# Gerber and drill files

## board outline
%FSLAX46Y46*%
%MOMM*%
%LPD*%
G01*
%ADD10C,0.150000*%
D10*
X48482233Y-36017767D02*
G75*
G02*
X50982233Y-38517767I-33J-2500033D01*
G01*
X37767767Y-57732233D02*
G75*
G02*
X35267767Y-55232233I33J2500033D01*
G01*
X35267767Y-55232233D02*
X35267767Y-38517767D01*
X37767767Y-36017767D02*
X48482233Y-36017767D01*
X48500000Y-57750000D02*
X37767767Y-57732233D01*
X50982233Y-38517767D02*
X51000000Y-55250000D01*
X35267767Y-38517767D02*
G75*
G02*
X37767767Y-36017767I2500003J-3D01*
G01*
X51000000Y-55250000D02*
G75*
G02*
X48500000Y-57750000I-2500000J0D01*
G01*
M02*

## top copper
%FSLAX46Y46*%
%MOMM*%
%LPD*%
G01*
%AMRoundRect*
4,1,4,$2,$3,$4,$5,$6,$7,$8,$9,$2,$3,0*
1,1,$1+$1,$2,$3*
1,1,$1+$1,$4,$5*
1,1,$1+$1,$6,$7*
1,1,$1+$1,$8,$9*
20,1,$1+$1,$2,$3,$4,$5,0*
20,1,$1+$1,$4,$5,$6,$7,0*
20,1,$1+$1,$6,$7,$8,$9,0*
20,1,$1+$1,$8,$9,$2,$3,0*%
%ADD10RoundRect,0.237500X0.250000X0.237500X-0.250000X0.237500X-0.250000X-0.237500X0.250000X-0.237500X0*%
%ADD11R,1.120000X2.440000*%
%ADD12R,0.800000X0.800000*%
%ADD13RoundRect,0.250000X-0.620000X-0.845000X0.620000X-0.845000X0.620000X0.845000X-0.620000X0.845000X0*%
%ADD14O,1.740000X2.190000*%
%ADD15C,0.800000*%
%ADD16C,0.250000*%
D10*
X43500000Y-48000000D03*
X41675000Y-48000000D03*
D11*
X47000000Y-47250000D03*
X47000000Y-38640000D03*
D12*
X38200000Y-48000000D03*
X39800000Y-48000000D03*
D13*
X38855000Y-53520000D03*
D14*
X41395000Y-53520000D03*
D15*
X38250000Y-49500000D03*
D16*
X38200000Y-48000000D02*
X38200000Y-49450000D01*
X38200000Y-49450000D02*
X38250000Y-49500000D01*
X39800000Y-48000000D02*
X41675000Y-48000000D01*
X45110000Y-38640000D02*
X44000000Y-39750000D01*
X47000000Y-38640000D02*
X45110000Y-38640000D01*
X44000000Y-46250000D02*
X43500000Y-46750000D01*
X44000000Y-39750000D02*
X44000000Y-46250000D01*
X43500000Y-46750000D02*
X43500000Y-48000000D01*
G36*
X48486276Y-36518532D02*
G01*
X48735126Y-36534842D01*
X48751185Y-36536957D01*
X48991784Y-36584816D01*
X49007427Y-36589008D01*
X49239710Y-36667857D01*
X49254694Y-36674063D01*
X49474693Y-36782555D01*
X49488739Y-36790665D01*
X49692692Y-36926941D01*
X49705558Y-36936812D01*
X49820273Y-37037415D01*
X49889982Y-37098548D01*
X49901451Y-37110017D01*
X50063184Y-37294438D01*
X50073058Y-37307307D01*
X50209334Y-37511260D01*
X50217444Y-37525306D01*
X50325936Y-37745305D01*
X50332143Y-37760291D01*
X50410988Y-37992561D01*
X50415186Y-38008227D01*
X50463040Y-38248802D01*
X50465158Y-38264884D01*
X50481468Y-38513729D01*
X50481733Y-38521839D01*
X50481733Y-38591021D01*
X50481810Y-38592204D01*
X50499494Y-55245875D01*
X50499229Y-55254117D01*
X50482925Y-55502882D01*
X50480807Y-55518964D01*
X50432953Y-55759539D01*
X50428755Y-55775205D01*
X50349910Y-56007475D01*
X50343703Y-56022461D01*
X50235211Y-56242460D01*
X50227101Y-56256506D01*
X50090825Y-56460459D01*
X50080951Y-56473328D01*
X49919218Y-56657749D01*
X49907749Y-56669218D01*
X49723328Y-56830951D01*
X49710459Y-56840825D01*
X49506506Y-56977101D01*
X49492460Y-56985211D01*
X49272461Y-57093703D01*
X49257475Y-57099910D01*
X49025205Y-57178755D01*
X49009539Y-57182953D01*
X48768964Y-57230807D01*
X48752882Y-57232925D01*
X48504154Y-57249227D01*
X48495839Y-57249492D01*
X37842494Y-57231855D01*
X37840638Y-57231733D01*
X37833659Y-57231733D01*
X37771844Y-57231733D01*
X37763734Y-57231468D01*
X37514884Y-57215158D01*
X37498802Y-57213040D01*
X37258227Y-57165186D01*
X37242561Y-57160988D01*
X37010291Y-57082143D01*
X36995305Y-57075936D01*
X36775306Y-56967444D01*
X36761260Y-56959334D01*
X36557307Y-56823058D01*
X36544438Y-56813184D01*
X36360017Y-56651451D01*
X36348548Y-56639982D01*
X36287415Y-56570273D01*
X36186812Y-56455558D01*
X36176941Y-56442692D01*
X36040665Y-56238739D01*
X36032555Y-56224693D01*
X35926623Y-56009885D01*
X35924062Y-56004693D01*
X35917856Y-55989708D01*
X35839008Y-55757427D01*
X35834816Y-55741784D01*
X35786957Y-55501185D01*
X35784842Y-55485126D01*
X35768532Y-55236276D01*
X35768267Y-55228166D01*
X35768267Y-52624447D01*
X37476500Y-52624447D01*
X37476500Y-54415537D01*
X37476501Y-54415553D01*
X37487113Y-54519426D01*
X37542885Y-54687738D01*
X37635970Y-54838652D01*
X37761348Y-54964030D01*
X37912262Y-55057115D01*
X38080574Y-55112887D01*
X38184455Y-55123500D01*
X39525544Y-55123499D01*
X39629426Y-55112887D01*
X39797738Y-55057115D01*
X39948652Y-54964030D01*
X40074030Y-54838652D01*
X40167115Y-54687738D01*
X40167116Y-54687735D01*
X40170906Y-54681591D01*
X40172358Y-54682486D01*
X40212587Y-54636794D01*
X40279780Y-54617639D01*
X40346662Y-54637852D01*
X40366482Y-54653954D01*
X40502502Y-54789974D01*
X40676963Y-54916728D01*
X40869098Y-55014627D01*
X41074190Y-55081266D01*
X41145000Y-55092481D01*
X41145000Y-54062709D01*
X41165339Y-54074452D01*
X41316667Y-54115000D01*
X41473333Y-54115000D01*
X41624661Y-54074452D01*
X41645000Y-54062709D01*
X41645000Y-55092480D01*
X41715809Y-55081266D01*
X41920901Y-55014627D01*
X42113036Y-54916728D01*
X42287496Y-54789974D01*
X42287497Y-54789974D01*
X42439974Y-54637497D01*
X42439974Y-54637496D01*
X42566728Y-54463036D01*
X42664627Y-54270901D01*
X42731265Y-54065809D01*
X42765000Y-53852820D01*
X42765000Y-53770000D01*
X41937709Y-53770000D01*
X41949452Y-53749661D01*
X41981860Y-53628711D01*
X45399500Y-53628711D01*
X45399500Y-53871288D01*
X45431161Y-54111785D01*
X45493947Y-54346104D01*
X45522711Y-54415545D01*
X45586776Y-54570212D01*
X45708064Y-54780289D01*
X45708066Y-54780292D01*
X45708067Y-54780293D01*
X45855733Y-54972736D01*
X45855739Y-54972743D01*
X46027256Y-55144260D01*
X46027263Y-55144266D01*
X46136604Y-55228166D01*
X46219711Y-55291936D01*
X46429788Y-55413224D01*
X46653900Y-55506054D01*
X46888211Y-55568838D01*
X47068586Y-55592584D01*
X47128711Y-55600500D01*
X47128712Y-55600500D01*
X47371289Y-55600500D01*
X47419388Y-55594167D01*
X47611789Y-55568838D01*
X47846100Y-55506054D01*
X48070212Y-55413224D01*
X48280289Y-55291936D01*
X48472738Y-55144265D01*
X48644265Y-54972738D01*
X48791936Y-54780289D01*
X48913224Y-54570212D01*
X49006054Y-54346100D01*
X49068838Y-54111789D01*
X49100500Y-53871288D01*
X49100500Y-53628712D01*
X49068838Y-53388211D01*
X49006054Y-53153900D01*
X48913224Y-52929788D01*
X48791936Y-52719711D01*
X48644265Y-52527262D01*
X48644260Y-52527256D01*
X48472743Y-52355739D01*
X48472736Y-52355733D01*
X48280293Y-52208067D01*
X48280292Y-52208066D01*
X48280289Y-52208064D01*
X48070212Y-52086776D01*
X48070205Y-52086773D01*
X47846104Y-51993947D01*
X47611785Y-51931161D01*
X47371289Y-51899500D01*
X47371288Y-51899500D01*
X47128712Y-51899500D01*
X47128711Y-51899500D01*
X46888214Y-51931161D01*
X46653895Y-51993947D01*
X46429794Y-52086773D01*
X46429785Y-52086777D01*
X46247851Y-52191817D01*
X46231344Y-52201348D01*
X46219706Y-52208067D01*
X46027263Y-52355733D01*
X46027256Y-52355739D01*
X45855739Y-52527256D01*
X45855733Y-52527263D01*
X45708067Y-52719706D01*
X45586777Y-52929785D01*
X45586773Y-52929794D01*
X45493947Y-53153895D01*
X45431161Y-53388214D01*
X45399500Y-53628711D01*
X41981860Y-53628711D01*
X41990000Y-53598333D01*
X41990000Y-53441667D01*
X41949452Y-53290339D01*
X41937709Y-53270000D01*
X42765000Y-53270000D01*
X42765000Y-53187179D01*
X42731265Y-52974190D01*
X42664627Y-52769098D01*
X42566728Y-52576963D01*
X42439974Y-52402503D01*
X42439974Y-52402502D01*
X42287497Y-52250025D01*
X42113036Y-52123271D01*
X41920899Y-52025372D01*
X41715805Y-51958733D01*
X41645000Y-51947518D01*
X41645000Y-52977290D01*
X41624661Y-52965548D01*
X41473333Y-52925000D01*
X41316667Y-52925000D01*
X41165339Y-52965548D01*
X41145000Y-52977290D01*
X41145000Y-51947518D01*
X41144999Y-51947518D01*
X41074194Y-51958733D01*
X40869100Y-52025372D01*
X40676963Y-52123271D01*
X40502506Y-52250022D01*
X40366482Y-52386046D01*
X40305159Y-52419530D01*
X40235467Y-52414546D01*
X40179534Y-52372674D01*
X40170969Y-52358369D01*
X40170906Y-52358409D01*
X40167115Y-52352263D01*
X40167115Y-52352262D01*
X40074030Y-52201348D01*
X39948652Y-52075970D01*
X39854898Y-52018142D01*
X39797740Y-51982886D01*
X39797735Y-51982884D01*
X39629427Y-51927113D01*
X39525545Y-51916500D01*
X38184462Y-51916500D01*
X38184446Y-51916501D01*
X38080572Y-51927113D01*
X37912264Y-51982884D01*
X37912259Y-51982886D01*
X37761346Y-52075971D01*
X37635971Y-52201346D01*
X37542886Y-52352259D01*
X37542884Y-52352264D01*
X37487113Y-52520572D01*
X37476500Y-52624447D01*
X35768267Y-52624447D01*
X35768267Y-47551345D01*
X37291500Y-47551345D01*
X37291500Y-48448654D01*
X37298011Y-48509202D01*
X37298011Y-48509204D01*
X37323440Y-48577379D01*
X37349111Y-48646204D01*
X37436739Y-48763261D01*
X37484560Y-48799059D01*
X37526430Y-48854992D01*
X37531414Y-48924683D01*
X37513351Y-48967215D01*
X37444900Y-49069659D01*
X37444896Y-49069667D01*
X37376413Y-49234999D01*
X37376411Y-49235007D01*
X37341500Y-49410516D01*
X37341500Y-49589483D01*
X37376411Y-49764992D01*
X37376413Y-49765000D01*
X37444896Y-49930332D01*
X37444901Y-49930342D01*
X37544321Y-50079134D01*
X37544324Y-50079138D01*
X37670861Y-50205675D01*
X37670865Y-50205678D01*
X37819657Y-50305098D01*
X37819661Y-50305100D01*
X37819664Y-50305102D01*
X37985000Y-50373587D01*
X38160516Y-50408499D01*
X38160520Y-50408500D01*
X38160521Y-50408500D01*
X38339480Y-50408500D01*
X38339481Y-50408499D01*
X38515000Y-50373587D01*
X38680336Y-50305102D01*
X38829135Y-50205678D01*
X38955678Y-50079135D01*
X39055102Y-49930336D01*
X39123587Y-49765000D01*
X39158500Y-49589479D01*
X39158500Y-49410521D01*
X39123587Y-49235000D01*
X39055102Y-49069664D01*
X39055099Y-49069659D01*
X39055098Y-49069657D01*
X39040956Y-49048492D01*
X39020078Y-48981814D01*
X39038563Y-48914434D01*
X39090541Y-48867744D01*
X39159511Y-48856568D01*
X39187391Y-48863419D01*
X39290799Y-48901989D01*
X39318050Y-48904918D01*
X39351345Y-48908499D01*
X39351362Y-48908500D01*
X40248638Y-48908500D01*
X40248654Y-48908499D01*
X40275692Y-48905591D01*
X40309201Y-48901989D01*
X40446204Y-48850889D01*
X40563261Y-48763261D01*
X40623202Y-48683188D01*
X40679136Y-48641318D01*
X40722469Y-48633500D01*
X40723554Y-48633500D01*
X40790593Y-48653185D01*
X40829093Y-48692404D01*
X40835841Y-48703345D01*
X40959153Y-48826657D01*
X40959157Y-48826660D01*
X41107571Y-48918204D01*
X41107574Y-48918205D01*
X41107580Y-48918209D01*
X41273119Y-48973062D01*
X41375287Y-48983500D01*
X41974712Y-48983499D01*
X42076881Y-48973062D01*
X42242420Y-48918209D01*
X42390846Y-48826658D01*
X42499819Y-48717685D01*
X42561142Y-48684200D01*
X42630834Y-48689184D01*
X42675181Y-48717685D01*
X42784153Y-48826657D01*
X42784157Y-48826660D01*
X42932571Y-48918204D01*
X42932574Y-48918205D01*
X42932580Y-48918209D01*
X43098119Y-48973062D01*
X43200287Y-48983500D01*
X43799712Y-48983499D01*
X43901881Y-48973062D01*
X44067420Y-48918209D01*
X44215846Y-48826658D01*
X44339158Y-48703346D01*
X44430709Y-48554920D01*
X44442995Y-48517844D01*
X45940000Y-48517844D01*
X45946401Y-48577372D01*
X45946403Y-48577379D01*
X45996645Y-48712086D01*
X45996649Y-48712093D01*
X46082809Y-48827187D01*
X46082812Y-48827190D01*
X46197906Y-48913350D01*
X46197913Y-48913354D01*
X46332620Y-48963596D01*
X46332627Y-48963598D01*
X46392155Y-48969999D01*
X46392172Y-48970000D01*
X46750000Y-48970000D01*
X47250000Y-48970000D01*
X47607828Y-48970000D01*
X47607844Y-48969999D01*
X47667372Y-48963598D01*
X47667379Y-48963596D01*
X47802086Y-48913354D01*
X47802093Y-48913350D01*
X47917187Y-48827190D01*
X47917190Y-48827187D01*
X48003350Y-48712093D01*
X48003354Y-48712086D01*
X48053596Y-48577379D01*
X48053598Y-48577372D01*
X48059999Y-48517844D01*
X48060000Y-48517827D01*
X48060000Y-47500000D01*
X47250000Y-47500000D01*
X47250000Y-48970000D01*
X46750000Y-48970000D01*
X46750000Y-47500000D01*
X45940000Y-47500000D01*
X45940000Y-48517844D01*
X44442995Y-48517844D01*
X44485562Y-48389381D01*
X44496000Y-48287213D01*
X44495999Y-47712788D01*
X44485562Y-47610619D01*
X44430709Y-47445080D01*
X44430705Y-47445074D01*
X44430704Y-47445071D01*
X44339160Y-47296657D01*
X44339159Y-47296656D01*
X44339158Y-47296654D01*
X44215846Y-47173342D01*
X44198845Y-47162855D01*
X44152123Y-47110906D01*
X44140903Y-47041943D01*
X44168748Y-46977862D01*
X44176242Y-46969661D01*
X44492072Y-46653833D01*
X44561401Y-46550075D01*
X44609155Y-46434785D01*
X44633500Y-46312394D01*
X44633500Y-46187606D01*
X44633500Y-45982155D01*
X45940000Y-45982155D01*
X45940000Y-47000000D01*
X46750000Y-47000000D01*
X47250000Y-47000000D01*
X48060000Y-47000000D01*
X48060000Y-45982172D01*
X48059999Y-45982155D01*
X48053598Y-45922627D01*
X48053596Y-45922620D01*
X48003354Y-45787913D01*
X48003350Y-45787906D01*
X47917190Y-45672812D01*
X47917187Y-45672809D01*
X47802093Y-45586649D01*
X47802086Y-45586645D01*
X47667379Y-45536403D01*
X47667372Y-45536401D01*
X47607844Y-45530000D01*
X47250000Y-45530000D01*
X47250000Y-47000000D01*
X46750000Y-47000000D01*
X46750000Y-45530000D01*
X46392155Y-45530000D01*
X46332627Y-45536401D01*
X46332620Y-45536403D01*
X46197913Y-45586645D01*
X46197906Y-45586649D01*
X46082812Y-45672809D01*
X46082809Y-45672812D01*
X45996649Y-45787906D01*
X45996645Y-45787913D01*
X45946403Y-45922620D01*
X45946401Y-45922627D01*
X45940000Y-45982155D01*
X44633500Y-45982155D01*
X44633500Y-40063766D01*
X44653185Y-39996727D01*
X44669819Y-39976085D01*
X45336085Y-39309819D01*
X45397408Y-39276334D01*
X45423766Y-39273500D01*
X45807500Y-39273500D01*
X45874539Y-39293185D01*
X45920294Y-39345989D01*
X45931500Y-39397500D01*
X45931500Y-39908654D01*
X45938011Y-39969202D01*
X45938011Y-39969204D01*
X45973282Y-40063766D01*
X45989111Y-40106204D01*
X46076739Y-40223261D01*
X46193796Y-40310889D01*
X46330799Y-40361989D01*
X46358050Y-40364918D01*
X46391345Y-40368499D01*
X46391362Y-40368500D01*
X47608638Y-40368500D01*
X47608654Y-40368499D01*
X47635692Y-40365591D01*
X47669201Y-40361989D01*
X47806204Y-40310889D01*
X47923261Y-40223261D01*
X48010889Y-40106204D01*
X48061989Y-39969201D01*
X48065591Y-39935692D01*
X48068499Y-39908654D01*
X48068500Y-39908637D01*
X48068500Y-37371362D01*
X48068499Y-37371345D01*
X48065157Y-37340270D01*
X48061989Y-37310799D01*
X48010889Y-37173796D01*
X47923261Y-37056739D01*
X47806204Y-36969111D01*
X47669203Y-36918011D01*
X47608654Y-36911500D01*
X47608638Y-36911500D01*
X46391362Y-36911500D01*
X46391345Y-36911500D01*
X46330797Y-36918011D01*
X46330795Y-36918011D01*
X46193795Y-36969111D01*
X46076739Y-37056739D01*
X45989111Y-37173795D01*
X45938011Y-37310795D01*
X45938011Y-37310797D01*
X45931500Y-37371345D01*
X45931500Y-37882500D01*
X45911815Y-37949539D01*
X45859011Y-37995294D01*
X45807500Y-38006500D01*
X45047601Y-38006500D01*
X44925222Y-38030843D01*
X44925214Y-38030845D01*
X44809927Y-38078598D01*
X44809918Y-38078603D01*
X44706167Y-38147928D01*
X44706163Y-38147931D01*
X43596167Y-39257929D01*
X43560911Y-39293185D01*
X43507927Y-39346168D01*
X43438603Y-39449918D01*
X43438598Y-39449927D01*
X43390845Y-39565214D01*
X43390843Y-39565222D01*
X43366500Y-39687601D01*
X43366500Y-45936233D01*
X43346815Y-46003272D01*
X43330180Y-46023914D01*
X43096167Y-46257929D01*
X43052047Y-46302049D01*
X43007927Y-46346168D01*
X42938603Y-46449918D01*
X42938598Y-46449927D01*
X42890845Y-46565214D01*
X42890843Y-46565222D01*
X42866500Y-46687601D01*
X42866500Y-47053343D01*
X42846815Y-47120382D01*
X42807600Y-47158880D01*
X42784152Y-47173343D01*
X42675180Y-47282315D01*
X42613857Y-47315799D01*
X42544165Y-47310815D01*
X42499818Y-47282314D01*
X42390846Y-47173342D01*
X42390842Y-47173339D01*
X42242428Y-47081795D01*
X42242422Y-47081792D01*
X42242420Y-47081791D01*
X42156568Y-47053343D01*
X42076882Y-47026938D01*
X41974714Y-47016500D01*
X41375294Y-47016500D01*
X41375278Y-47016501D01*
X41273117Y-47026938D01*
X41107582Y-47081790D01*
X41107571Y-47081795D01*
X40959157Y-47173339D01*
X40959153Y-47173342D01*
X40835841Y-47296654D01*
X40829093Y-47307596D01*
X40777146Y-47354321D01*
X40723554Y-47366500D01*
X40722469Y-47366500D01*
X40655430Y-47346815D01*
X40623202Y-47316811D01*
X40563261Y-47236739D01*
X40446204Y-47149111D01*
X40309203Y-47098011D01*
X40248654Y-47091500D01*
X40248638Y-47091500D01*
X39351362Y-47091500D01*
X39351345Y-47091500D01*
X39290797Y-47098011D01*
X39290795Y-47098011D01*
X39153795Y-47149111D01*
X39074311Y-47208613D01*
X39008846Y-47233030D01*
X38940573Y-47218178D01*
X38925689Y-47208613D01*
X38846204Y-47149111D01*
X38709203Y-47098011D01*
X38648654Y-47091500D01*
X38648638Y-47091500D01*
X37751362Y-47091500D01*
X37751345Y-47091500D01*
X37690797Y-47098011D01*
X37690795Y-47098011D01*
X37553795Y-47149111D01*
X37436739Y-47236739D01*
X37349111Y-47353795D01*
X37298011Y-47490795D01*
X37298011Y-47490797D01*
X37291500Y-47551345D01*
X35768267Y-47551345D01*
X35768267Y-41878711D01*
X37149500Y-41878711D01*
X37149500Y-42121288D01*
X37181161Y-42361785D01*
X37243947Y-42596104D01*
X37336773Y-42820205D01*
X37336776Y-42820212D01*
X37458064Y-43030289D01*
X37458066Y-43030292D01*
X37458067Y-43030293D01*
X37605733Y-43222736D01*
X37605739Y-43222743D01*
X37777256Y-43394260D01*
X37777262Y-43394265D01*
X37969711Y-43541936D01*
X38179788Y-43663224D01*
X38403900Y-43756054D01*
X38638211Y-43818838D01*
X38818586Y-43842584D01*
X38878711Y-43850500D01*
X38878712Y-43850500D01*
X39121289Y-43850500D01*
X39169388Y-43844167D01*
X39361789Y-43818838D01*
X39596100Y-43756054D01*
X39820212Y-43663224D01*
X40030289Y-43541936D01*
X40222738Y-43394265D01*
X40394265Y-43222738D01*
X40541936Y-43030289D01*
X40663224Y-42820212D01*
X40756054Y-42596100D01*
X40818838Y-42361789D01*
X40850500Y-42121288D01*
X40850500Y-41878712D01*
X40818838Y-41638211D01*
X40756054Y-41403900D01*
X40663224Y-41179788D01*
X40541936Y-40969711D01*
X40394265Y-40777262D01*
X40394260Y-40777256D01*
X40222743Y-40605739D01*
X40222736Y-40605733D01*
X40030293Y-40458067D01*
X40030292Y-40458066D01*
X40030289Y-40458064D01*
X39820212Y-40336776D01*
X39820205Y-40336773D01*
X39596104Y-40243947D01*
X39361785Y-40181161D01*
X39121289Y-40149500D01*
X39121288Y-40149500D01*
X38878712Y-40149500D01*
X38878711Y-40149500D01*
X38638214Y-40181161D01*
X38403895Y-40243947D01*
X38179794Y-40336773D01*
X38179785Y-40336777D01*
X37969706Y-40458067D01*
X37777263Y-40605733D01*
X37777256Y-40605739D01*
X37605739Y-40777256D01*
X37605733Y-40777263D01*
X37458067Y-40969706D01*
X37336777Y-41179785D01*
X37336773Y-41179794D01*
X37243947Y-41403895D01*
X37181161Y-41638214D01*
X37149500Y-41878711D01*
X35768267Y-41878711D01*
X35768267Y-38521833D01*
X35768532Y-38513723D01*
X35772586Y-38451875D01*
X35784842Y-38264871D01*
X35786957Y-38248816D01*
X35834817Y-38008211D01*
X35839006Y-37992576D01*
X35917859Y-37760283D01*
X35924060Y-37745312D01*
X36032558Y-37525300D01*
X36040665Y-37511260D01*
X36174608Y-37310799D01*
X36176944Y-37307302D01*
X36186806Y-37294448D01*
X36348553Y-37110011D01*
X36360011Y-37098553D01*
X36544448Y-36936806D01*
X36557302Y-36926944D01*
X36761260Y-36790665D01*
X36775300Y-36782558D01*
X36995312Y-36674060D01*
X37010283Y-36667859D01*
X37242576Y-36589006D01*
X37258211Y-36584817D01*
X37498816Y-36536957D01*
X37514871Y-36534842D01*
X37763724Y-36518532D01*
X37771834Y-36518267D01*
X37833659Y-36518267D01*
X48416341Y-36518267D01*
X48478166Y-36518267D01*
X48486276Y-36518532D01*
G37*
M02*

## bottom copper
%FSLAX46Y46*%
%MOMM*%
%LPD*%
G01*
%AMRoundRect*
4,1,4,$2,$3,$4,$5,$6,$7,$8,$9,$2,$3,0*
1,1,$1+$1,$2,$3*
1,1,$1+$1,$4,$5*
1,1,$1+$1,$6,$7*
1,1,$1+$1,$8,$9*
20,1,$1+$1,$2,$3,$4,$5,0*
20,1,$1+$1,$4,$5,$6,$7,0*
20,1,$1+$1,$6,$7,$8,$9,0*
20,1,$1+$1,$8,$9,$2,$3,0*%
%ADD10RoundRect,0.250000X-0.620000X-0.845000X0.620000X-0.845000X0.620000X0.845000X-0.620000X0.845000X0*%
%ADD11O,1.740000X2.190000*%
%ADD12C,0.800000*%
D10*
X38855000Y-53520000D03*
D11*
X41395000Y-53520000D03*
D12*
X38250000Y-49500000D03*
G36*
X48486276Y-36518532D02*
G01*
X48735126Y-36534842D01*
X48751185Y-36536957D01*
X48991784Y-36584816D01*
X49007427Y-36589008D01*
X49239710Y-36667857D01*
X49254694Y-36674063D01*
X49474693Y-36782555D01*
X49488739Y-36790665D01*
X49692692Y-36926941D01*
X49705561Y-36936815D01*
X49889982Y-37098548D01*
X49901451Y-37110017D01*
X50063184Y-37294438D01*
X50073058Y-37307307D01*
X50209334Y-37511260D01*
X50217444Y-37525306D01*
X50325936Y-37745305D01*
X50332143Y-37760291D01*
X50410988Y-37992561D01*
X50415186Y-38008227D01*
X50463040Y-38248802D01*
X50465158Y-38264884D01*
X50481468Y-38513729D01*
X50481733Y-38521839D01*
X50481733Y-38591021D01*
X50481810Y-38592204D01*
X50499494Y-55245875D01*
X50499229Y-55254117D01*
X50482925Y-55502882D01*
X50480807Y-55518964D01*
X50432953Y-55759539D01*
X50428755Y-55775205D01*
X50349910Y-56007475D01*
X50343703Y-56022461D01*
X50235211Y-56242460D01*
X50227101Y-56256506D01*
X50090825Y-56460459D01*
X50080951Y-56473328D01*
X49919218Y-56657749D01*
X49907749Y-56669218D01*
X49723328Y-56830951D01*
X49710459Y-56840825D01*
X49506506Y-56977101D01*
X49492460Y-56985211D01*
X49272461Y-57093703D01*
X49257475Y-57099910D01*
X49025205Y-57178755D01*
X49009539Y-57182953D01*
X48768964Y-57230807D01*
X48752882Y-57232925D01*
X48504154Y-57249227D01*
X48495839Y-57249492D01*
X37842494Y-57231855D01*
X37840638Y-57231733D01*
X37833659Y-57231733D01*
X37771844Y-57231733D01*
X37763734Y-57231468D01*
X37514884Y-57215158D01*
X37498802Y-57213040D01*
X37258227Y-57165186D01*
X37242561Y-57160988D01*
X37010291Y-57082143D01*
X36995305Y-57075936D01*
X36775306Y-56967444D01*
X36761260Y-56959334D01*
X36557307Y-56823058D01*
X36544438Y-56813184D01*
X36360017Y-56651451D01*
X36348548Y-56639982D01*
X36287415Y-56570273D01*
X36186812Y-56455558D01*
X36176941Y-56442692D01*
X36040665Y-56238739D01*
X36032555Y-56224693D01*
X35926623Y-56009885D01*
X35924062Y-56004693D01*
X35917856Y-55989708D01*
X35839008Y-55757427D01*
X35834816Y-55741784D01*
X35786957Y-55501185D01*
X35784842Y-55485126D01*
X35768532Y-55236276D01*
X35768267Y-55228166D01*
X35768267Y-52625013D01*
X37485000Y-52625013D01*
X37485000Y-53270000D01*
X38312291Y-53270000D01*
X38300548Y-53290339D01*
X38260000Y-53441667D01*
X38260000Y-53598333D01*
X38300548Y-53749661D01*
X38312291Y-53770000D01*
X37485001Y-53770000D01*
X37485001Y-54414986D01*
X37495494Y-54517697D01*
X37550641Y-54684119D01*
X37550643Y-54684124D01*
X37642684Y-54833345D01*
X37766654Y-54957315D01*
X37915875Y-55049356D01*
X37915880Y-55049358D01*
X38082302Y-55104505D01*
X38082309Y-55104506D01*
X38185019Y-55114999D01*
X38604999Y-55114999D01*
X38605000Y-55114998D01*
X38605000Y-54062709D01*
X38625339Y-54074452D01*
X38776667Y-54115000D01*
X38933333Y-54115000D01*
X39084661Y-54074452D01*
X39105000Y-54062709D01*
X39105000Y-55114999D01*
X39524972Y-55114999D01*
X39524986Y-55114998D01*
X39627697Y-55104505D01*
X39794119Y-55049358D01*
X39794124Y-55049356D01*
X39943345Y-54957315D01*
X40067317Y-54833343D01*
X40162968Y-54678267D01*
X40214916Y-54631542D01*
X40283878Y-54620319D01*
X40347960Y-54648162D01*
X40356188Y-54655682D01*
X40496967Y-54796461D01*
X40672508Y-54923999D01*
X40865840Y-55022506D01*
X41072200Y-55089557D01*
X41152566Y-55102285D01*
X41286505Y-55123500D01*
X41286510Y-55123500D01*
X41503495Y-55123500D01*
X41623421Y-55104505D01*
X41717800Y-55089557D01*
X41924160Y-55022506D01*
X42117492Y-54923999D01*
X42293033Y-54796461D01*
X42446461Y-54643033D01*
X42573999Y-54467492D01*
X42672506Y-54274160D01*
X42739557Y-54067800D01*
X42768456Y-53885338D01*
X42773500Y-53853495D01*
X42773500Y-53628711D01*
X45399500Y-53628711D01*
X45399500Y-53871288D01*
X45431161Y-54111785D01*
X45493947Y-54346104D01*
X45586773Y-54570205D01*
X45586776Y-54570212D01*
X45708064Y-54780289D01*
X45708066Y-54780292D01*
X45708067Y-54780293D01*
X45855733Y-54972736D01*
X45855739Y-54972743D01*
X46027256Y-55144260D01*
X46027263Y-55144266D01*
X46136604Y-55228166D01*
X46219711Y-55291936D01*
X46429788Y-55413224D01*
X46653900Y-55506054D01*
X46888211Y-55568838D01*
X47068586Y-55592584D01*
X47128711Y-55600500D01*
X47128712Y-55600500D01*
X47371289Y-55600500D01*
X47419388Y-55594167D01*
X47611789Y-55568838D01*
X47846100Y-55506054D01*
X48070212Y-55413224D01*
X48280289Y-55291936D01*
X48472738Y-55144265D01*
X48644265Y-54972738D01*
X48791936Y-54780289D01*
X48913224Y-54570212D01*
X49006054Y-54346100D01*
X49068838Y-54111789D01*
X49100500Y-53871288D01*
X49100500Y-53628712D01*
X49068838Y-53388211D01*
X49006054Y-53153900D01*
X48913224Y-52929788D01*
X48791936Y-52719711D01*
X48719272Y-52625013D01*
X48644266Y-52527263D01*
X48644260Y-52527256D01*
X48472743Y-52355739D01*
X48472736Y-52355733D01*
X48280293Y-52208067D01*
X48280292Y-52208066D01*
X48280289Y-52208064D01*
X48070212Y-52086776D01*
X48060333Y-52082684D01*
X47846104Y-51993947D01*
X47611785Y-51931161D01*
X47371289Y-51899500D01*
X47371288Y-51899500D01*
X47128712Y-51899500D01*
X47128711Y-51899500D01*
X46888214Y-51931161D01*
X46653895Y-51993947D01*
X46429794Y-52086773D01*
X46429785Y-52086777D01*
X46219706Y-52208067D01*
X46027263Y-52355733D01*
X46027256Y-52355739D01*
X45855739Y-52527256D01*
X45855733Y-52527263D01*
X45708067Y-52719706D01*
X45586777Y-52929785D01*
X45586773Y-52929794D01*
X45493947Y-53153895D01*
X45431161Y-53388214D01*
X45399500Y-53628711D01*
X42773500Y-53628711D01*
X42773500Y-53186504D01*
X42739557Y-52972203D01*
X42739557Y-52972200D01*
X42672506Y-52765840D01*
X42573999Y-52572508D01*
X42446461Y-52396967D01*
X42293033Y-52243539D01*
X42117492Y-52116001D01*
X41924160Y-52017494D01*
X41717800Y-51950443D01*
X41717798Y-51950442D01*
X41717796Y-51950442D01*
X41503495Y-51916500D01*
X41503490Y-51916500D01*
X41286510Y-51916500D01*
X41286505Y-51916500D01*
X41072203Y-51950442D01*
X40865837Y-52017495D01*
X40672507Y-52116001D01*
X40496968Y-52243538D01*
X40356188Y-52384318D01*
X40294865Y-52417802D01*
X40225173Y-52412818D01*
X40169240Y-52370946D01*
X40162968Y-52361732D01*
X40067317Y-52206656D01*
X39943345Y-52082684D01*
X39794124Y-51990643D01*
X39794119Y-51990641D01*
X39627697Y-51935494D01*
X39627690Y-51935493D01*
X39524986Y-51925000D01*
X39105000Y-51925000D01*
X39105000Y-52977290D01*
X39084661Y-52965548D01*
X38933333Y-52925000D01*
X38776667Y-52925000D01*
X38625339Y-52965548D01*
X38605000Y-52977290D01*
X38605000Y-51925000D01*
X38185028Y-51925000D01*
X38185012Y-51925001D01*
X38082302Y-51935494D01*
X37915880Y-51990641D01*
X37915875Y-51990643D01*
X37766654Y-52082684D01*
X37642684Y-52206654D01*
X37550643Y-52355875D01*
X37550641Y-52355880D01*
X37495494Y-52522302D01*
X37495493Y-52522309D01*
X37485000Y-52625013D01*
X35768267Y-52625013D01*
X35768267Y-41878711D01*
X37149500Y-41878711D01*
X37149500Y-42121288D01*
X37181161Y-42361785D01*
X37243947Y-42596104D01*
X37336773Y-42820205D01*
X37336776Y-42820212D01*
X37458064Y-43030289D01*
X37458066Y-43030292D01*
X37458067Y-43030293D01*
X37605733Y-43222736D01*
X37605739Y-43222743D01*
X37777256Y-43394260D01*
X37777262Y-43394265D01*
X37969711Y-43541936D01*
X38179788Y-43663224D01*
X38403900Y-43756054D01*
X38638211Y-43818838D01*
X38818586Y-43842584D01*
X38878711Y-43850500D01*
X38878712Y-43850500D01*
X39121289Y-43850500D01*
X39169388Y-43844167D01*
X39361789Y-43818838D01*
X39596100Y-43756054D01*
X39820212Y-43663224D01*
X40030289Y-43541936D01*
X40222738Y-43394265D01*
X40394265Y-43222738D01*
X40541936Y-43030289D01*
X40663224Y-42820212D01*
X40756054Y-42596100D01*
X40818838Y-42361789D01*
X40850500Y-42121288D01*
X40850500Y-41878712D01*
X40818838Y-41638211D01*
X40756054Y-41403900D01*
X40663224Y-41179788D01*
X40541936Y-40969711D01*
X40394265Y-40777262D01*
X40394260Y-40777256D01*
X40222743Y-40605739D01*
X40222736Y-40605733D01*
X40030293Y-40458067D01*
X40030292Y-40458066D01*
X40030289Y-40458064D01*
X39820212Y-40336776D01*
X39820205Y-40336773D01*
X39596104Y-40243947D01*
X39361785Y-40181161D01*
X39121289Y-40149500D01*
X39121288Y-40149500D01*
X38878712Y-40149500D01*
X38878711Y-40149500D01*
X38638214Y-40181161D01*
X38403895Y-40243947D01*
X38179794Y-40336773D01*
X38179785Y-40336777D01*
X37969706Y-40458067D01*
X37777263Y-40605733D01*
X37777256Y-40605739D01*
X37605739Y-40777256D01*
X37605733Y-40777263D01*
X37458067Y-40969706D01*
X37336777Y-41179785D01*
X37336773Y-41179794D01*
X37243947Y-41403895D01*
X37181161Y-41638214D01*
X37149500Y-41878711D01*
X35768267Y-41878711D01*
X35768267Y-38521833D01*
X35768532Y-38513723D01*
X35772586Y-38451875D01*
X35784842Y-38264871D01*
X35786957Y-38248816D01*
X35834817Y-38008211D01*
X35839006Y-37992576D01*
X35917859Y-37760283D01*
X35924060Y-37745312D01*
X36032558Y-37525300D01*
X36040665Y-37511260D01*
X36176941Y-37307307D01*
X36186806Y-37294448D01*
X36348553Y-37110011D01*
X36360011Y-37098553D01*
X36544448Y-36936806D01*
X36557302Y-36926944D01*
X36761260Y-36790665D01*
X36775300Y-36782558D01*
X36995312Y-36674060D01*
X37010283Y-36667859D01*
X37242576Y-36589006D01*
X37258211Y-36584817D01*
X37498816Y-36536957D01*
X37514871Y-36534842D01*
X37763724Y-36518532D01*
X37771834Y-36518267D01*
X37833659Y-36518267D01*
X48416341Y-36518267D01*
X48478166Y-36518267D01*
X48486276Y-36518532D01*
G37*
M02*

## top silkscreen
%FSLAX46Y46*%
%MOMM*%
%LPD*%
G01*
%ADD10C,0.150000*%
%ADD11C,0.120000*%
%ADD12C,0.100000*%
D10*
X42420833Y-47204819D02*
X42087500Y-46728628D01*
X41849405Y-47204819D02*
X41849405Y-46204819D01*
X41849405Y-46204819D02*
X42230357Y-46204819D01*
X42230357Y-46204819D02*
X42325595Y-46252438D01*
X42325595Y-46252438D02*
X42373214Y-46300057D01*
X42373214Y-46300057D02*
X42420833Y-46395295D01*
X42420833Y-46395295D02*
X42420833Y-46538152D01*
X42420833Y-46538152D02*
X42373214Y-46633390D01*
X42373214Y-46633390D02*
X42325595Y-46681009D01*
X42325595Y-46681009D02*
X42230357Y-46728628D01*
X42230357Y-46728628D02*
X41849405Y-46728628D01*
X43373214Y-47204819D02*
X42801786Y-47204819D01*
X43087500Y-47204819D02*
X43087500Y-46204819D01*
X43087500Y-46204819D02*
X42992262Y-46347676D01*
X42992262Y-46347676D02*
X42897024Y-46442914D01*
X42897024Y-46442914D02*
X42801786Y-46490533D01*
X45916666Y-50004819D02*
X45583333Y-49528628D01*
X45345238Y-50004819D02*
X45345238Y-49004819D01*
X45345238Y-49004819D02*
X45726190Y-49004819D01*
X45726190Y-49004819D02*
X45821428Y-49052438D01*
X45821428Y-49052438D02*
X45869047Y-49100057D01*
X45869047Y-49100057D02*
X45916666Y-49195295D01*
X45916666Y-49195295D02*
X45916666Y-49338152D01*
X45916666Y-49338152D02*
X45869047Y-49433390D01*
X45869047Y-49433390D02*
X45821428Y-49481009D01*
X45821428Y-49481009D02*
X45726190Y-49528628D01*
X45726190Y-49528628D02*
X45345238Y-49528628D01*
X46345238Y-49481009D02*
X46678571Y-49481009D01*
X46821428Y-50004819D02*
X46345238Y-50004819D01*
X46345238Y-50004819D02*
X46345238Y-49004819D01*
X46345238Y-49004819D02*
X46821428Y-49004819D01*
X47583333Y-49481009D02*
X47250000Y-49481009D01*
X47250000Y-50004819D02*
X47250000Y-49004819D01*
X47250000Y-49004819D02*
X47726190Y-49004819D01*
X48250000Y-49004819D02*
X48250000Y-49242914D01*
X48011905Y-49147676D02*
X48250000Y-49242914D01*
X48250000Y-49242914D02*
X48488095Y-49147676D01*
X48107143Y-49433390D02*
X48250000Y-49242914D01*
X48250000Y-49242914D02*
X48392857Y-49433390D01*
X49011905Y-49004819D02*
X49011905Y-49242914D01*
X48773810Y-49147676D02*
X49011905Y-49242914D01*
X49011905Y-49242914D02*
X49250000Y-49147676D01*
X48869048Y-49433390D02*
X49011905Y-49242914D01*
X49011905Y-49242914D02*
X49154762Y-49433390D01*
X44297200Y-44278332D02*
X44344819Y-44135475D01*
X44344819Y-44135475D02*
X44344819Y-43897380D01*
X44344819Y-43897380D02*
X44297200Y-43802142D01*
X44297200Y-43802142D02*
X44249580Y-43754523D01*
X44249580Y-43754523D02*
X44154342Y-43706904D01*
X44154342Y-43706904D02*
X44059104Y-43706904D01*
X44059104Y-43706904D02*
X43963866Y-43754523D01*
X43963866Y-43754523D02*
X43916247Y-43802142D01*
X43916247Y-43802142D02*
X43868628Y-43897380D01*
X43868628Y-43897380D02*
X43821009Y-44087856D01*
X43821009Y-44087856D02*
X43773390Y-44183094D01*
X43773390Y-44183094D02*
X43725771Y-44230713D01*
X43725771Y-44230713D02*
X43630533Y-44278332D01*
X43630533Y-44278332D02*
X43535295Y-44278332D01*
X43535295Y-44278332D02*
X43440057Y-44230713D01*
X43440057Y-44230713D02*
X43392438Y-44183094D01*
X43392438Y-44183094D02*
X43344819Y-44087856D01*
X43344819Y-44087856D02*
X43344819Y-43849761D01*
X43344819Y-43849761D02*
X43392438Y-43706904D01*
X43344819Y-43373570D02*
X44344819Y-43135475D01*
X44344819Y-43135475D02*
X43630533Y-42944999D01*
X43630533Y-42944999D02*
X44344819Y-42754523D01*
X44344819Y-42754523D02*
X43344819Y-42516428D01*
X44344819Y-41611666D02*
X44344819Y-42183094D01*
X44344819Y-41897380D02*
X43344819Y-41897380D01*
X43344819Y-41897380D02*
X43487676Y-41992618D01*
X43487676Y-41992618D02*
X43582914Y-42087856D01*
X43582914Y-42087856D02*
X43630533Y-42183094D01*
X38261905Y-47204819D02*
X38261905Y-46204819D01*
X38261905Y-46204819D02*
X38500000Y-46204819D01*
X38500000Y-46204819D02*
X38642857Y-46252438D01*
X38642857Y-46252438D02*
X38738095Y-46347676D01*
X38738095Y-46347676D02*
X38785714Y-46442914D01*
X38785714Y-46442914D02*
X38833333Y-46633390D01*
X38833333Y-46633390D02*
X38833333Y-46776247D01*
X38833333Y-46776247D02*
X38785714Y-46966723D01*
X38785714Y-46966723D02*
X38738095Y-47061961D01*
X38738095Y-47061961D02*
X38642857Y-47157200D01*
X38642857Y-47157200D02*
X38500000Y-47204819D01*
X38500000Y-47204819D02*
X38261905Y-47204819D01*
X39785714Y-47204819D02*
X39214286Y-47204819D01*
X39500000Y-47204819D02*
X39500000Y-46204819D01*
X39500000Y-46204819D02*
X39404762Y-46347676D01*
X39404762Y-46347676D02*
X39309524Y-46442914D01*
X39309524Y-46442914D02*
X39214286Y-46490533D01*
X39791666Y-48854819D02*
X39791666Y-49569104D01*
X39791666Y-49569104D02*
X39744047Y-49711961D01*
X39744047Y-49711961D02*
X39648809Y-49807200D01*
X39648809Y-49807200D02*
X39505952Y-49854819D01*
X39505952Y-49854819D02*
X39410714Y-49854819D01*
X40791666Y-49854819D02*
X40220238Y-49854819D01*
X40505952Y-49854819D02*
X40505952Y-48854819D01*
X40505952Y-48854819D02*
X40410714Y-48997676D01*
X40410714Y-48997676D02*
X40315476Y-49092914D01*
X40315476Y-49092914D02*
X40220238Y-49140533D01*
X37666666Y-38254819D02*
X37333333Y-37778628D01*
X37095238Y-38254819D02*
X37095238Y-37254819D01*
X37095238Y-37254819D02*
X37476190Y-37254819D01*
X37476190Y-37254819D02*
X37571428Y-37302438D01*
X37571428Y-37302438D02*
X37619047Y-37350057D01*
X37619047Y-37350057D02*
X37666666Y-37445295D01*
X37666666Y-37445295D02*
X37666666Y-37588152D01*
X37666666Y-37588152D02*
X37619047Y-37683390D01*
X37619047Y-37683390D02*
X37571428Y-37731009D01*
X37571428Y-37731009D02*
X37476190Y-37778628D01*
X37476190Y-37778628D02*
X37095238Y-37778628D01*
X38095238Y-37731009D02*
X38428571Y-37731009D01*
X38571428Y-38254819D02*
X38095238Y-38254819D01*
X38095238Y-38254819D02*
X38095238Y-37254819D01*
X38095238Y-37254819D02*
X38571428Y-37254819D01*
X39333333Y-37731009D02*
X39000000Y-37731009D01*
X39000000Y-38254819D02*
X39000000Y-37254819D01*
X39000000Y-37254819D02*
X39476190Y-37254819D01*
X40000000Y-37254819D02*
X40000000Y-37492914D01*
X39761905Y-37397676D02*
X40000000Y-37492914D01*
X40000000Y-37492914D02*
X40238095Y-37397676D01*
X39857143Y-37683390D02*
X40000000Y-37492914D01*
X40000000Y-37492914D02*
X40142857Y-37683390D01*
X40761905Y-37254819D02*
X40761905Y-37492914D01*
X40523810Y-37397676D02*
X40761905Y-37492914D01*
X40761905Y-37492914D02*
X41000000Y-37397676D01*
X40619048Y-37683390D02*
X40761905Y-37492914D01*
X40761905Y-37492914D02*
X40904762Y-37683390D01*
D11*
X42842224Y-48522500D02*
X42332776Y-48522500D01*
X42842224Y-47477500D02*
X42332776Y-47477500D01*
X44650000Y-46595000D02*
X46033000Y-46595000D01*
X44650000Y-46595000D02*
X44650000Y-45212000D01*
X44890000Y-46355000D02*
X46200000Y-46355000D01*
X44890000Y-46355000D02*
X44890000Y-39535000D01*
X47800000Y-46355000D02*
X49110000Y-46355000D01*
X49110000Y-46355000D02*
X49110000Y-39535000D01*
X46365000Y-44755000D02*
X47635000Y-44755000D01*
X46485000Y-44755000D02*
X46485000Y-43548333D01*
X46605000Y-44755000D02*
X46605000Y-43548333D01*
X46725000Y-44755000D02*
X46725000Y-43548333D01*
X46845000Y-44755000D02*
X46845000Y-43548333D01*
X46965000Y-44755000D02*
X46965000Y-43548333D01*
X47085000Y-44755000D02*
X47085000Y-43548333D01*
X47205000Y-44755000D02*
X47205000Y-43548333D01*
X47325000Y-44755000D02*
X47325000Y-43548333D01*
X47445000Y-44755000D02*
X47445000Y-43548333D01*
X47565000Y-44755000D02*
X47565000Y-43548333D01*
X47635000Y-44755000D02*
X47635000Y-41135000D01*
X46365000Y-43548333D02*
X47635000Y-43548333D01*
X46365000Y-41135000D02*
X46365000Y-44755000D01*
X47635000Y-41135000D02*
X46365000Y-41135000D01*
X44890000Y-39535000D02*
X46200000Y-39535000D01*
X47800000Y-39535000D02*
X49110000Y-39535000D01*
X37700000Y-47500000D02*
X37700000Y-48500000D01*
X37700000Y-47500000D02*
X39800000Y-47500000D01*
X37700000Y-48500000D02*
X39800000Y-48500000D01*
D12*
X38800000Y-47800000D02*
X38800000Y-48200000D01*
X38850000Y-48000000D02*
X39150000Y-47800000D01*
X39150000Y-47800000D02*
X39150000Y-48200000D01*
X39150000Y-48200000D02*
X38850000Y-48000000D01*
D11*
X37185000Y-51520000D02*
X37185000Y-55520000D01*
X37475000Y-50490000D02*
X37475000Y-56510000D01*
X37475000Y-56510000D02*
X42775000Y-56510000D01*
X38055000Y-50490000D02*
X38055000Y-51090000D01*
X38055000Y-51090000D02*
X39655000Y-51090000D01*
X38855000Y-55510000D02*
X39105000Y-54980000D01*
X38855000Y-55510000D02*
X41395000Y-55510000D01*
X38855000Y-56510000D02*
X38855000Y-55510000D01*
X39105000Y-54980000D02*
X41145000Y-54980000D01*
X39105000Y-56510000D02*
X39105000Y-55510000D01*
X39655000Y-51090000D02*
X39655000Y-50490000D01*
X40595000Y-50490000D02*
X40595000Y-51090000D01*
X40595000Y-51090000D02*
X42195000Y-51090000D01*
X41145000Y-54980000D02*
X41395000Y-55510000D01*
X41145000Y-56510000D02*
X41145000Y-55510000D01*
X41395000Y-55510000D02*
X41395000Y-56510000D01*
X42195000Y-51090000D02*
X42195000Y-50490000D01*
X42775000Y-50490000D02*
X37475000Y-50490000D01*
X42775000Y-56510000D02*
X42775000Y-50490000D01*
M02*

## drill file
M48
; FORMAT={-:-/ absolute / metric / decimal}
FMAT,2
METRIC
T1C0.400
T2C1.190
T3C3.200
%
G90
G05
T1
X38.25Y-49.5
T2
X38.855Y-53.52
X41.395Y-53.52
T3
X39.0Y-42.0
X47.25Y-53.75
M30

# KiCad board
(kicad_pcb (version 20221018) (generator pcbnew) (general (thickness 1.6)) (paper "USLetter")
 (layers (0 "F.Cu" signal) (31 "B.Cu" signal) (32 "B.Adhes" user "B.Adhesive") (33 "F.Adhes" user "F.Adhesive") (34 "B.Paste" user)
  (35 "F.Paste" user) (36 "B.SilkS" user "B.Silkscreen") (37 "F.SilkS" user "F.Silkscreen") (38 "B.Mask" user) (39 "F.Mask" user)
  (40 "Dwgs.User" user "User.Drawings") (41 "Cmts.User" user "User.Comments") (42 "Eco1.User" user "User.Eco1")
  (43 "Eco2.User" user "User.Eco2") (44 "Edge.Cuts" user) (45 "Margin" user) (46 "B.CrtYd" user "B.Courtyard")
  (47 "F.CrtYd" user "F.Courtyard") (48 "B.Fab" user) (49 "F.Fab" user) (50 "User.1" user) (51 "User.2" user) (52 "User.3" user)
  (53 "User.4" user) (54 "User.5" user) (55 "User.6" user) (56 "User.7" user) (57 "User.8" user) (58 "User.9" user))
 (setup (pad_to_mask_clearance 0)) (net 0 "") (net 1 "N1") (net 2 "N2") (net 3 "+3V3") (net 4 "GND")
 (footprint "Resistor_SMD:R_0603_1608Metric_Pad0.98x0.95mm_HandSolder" (layer "F.Cu") (at 42.5875 48 180)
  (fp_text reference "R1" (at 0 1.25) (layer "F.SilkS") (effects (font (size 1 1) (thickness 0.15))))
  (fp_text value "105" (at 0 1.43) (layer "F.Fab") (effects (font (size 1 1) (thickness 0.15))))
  (fp_line (start -0.254724 -0.5225) (end 0.254724 -0.5225) (stroke (width 0.12) (type solid)) (layer "F.SilkS"))
  (fp_line (start -0.254724 0.5225) (end 0.254724 0.5225) (stroke (width 0.12) (type solid)) (layer "F.SilkS"))
  (pad "1" smd roundrect (at -0.9125 0 180) (size 0.975 0.95) (layers "F.Cu" "F.Paste" "F.Mask") (roundrect_rratio 0.25) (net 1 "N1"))
  (pad "2" smd roundrect (at 0.9125 0 180) (size 0.975 0.95) (layers "F.Cu" "F.Paste" "F.Mask") (roundrect_rratio 0.25) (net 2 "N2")))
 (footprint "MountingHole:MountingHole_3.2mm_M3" (layer "F.Cu") (at 47.25 53.75)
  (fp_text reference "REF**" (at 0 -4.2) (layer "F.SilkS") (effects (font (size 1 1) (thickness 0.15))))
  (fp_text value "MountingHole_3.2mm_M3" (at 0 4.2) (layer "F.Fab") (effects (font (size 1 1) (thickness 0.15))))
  (pad "" np_thru_hole circle (at 0 0) (size 3.2 3.2) (drill 3.2) (layers "F&B.Cu" "*.Mask")))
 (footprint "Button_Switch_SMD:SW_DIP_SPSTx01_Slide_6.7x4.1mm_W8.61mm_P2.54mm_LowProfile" (layer "F.Cu") (at 47 42.945 90)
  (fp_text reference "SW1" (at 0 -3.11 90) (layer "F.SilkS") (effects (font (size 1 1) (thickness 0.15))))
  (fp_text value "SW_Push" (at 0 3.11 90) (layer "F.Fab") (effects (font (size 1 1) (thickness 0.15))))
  (fp_line (start -3.65 -2.35) (end -3.65 -0.967) (stroke (width 0.12) (type solid)) (layer "F.SilkS"))
  (fp_line (start -3.65 -2.35) (end -2.267 -2.35) (stroke (width 0.12) (type solid)) (layer "F.SilkS"))
  (fp_line (start -3.41 -2.11) (end -3.41 -0.8) (stroke (width 0.12) (type solid)) (layer "F.SilkS"))
  (fp_line (start -3.41 -2.11) (end 3.41 -2.11) (stroke (width 0.12) (type solid)) (layer "F.SilkS"))
  (fp_line (start -3.41 0.8) (end -3.41 2.11) (stroke (width 0.12) (type solid)) (layer "F.SilkS"))
  (fp_line (start -3.41 2.11) (end 3.41 2.11) (stroke (width 0.12) (type solid)) (layer "F.SilkS"))
  (fp_line (start -1.81 -0.635) (end -1.81 0.635) (stroke (width 0.12) (type solid)) (layer "F.SilkS"))
  (fp_line (start -1.81 -0.515) (end -0.603333 -0.515) (stroke (width 0.12) (type solid)) (layer "F.SilkS"))
  (fp_line (start -1.81 -0.395) (end -0.603333 -0.395) (stroke (width 0.12) (type solid)) (layer "F.SilkS"))
  (fp_line (start -1.81 -0.275) (end -0.603333 -0.275) (stroke (width 0.12) (type solid)) (layer "F.SilkS"))
  (fp_line (start -1.81 -0.155) (end -0.603333 -0.155) (stroke (width 0.12) (type solid)) (layer "F.SilkS"))
  (fp_line (start -1.81 -0.035) (end -0.603333 -0.035) (stroke (width 0.12) (type solid)) (layer "F.SilkS"))
  (fp_line (start -1.81 0.085) (end -0.603333 0.085) (stroke (width 0.12) (type solid)) (layer "F.SilkS"))
  (fp_line (start -1.81 0.205) (end -0.603333 0.205) (stroke (width 0.12) (type solid)) (layer "F.SilkS"))
  (fp_line (start -1.81 0.325) (end -0.603333 0.325) (stroke (width 0.12) (type solid)) (layer "F.SilkS"))
  (fp_line (start -1.81 0.445) (end -0.603333 0.445) (stroke (width 0.12) (type solid)) (layer "F.SilkS"))
  (fp_line (start -1.81 0.565) (end -0.603333 0.565) (stroke (width 0.12) (type solid)) (layer "F.SilkS"))
  (fp_line (start -1.81 0.635) (end 1.81 0.635) (stroke (width 0.12) (type solid)) (layer "F.SilkS"))
  (fp_line (start -0.603333 -0.635) (end -0.603333 0.635) (stroke (width 0.12) (type solid)) (layer "F.SilkS"))
  (fp_line (start 1.81 -0.635) (end -1.81 -0.635) (stroke (width 0.12) (type solid)) (layer "F.SilkS"))
  (fp_line (start 1.81 0.635) (end 1.81 -0.635) (stroke (width 0.12) (type solid)) (layer "F.SilkS"))
  (fp_line (start 3.41 -2.11) (end 3.41 -0.8) (stroke (width 0.12) (type solid)) (layer "F.SilkS"))
  (fp_line (start 3.41 0.8) (end 3.41 2.11) (stroke (width 0.12) (type solid)) (layer "F.SilkS"))
  (pad "1" smd rect (at -4.305 0 90) (size 2.44 1.12) (layers "F.Cu" "F.Paste" "F.Mask") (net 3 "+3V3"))
  (pad "2" smd rect (at 4.305 0 90) (size 2.44 1.12) (layers "F.Cu" "F.Paste" "F.Mask") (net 1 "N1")))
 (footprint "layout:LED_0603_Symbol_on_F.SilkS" (layer "F.Cu") (at 39 48)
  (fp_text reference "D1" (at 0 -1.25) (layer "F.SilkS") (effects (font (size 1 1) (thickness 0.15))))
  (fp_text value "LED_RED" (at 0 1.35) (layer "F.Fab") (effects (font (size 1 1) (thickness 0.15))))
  (fp_line (start -1.3 -0.5) (end -1.3 0.5) (stroke (width 0.12) (type solid)) (layer "F.SilkS"))
  (fp_line (start -1.3 -0.5) (end 0.8 -0.5) (stroke (width 0.12) (type solid)) (layer "F.SilkS"))
  (fp_line (start -1.3 0.5) (end 0.8 0.5) (stroke (width 0.12) (type solid)) (layer "F.SilkS"))
  (fp_line (start -0.2 -0.2) (end -0.2 0.2) (stroke (width 0.1) (type solid)) (layer "F.SilkS"))
  (fp_line (start -0.15 0) (end 0.15 -0.2) (stroke (width 0.1) (type solid)) (layer "F.SilkS"))
  (fp_line (start 0.15 -0.2) (end 0.15 0.2) (stroke (width 0.1) (type solid)) (layer "F.SilkS"))
  (fp_line (start 0.15 0.2) (end -0.15 0) (stroke (width 0.1) (type solid)) (layer "F.SilkS"))
  (pad "1" smd rect (at -0.8 0 180) (size 0.8 0.8) (layers "F.Cu" "F.Paste" "F.Mask") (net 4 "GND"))
  (pad "2" smd rect (at 0.8 0 180) (size 0.8 0.8) (layers "F.Cu" "F.Paste" "F.Mask") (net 2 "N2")))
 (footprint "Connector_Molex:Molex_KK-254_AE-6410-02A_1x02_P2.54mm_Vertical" (layer "F.Cu") (at 38.855 53.52)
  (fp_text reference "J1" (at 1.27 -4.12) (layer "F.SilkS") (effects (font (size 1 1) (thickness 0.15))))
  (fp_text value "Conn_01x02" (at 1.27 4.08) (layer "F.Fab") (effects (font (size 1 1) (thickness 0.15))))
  (fp_line (start -1.67 -2) (end -1.67 2) (stroke (width 0.12) (type solid)) (layer "F.SilkS"))
  (fp_line (start -1.38 -3.03) (end -1.38 2.99) (stroke (width 0.12) (type solid)) (layer "F.SilkS"))
  (fp_line (start -1.38 2.99) (end 3.92 2.99) (stroke (width 0.12) (type solid)) (layer "F.SilkS"))
  (fp_line (start -0.8 -3.03) (end -0.8 -2.43) (stroke (width 0.12) (type solid)) (layer "F.SilkS"))
  (fp_line (start -0.8 -2.43) (end 0.8 -2.43) (stroke (width 0.12) (type solid)) (layer "F.SilkS"))
  (fp_line (start 0 1.99) (end 0.25 1.46) (stroke (width 0.12) (type solid)) (layer "F.SilkS"))
  (fp_line (start 0 1.99) (end 2.54 1.99) (stroke (width 0.12) (type solid)) (layer "F.SilkS"))
  (fp_line (start 0 2.99) (end 0 1.99) (stroke (width 0.12) (type solid)) (layer "F.SilkS"))
  (fp_line (start 0.25 1.46) (end 2.29 1.46) (stroke (width 0.12) (type solid)) (layer "F.SilkS"))
  (fp_line (start 0.25 2.99) (end 0.25 1.99) (stroke (width 0.12) (type solid)) (layer "F.SilkS"))
  (fp_line (start 0.8 -2.43) (end 0.8 -3.03) (stroke (width 0.12) (type solid)) (layer "F.SilkS"))
  (fp_line (start 1.74 -3.03) (end 1.74 -2.43) (stroke (width 0.12) (type solid)) (layer "F.SilkS"))
  (fp_line (start 1.74 -2.43) (end 3.34 -2.43) (stroke (width 0.12) (type solid)) (layer "F.SilkS"))
  (fp_line (start 2.29 1.46) (end 2.54 1.99) (stroke (width 0.12) (type solid)) (layer "F.SilkS"))
  (fp_line (start 2.29 2.99) (end 2.29 1.99) (stroke (width 0.12) (type solid)) (layer "F.SilkS"))
  (fp_line (start 2.54 1.99) (end 2.54 2.99) (stroke (width 0.12) (type solid)) (layer "F.SilkS"))
  (fp_line (start 3.34 -2.43) (end 3.34 -3.03) (stroke (width 0.12) (type solid)) (layer "F.SilkS"))
  (fp_line (start 3.92 -3.03) (end -1.38 -3.03) (stroke (width 0.12) (type solid)) (layer "F.SilkS"))
  (fp_line (start 3.92 2.99) (end 3.92 -3.03) (stroke (width 0.12) (type solid)) (layer "F.SilkS"))
  (pad "1" thru_hole roundrect (at 0 0) (size 1.74 2.19) (drill 1.19) (layers "*.Cu" "*.Mask") (roundrect_rratio 0.143678) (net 4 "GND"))
  (pad "2" thru_hole oval (at 2.54 0) (size 1.74 2.19) (drill 1.19) (layers "*.Cu" "*.Mask") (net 3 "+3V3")))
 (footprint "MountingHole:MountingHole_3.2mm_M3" (layer "F.Cu") (at 39 42)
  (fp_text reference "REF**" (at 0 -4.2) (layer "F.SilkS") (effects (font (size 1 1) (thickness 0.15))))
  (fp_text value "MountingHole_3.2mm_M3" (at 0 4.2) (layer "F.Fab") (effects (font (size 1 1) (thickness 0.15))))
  (pad "" np_thru_hole circle (at 0 0) (size 3.2 3.2) (drill 3.2) (layers "*.Cu" "*.Mask")))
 (gr_arc (start 48.482233 36.017767) (mid 50.249999 36.75) (end 50.982233 38.517767) (stroke (width 0.15) (type default))
  (layer "Edge.Cuts"))
 (gr_arc (start 37.767767 57.732233) (mid 36.000001 57) (end 35.267767 55.232233) (stroke (width 0.15) (type default)) (layer "Edge.Cuts"))
 (gr_line (start 35.267767 55.232233) (end 35.267767 38.517767) (stroke (width 0.15) (type default)) (layer "Edge.Cuts"))
 (gr_line (start 37.767767 36.017767) (end 48.482233 36.017767) (stroke (width 0.15) (type default)) (layer "Edge.Cuts"))
 (gr_line (start 48.5 57.75) (end 37.767767 57.732233) (stroke (width 0.15) (type default)) (layer "Edge.Cuts"))
 (gr_line (start 50.982233 38.517767) (end 51 55.25) (stroke (width 0.15) (type default)) (layer "Edge.Cuts"))
 (gr_arc (start 35.267767 38.517767) (mid 36 36.750001) (end 37.767767 36.017767) (stroke (width 0.15) (type default)) (layer "Edge.Cuts"))
 (gr_arc (start 51 55.25) (mid 50.267767 57.017766) (end 48.5 57.75) (stroke (width 0.15) (type default)) (layer "Edge.Cuts"))
 (segment (start 38.2 48) (end 38.2 49.45) (width 0.25) (layer "F.Cu") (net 4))
 (segment (start 38.2 49.45) (end 38.25 49.5) (width 0.25) (layer "F.Cu") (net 4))
 (via (at 38.25 49.5) (size 0.8) (drill 0.4) (layers "F.Cu" "B.Cu") (free) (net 4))
 (segment (start 39.8 48) (end 41.675 48) (width 0.25) (layer "F.Cu") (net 2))
 (segment (start 45.11 38.64) (end 44 39.75) (width 0.25) (layer "F.Cu") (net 1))
 (segment (start 47 38.64) (end 45.11 38.64) (width 0.25) (layer "F.Cu") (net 1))
 (segment (start 44 46.25) (end 43.5 46.75) (width 0.25) (layer "F.Cu") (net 1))
 (segment (start 44 39.75) (end 44 46.25) (width 0.25) (layer "F.Cu") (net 1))
 (segment (start 43.5 46.75) (end 43.5 48) (width 0.25) (layer "F.Cu") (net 1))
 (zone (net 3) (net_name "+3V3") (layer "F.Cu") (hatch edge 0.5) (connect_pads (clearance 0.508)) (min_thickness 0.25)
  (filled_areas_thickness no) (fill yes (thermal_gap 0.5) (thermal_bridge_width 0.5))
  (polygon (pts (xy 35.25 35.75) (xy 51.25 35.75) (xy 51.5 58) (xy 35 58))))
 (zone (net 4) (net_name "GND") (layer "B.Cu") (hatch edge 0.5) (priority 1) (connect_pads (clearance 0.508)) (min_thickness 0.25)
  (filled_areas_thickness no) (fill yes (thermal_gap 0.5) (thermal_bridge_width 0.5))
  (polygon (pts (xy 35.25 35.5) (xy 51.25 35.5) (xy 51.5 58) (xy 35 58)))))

